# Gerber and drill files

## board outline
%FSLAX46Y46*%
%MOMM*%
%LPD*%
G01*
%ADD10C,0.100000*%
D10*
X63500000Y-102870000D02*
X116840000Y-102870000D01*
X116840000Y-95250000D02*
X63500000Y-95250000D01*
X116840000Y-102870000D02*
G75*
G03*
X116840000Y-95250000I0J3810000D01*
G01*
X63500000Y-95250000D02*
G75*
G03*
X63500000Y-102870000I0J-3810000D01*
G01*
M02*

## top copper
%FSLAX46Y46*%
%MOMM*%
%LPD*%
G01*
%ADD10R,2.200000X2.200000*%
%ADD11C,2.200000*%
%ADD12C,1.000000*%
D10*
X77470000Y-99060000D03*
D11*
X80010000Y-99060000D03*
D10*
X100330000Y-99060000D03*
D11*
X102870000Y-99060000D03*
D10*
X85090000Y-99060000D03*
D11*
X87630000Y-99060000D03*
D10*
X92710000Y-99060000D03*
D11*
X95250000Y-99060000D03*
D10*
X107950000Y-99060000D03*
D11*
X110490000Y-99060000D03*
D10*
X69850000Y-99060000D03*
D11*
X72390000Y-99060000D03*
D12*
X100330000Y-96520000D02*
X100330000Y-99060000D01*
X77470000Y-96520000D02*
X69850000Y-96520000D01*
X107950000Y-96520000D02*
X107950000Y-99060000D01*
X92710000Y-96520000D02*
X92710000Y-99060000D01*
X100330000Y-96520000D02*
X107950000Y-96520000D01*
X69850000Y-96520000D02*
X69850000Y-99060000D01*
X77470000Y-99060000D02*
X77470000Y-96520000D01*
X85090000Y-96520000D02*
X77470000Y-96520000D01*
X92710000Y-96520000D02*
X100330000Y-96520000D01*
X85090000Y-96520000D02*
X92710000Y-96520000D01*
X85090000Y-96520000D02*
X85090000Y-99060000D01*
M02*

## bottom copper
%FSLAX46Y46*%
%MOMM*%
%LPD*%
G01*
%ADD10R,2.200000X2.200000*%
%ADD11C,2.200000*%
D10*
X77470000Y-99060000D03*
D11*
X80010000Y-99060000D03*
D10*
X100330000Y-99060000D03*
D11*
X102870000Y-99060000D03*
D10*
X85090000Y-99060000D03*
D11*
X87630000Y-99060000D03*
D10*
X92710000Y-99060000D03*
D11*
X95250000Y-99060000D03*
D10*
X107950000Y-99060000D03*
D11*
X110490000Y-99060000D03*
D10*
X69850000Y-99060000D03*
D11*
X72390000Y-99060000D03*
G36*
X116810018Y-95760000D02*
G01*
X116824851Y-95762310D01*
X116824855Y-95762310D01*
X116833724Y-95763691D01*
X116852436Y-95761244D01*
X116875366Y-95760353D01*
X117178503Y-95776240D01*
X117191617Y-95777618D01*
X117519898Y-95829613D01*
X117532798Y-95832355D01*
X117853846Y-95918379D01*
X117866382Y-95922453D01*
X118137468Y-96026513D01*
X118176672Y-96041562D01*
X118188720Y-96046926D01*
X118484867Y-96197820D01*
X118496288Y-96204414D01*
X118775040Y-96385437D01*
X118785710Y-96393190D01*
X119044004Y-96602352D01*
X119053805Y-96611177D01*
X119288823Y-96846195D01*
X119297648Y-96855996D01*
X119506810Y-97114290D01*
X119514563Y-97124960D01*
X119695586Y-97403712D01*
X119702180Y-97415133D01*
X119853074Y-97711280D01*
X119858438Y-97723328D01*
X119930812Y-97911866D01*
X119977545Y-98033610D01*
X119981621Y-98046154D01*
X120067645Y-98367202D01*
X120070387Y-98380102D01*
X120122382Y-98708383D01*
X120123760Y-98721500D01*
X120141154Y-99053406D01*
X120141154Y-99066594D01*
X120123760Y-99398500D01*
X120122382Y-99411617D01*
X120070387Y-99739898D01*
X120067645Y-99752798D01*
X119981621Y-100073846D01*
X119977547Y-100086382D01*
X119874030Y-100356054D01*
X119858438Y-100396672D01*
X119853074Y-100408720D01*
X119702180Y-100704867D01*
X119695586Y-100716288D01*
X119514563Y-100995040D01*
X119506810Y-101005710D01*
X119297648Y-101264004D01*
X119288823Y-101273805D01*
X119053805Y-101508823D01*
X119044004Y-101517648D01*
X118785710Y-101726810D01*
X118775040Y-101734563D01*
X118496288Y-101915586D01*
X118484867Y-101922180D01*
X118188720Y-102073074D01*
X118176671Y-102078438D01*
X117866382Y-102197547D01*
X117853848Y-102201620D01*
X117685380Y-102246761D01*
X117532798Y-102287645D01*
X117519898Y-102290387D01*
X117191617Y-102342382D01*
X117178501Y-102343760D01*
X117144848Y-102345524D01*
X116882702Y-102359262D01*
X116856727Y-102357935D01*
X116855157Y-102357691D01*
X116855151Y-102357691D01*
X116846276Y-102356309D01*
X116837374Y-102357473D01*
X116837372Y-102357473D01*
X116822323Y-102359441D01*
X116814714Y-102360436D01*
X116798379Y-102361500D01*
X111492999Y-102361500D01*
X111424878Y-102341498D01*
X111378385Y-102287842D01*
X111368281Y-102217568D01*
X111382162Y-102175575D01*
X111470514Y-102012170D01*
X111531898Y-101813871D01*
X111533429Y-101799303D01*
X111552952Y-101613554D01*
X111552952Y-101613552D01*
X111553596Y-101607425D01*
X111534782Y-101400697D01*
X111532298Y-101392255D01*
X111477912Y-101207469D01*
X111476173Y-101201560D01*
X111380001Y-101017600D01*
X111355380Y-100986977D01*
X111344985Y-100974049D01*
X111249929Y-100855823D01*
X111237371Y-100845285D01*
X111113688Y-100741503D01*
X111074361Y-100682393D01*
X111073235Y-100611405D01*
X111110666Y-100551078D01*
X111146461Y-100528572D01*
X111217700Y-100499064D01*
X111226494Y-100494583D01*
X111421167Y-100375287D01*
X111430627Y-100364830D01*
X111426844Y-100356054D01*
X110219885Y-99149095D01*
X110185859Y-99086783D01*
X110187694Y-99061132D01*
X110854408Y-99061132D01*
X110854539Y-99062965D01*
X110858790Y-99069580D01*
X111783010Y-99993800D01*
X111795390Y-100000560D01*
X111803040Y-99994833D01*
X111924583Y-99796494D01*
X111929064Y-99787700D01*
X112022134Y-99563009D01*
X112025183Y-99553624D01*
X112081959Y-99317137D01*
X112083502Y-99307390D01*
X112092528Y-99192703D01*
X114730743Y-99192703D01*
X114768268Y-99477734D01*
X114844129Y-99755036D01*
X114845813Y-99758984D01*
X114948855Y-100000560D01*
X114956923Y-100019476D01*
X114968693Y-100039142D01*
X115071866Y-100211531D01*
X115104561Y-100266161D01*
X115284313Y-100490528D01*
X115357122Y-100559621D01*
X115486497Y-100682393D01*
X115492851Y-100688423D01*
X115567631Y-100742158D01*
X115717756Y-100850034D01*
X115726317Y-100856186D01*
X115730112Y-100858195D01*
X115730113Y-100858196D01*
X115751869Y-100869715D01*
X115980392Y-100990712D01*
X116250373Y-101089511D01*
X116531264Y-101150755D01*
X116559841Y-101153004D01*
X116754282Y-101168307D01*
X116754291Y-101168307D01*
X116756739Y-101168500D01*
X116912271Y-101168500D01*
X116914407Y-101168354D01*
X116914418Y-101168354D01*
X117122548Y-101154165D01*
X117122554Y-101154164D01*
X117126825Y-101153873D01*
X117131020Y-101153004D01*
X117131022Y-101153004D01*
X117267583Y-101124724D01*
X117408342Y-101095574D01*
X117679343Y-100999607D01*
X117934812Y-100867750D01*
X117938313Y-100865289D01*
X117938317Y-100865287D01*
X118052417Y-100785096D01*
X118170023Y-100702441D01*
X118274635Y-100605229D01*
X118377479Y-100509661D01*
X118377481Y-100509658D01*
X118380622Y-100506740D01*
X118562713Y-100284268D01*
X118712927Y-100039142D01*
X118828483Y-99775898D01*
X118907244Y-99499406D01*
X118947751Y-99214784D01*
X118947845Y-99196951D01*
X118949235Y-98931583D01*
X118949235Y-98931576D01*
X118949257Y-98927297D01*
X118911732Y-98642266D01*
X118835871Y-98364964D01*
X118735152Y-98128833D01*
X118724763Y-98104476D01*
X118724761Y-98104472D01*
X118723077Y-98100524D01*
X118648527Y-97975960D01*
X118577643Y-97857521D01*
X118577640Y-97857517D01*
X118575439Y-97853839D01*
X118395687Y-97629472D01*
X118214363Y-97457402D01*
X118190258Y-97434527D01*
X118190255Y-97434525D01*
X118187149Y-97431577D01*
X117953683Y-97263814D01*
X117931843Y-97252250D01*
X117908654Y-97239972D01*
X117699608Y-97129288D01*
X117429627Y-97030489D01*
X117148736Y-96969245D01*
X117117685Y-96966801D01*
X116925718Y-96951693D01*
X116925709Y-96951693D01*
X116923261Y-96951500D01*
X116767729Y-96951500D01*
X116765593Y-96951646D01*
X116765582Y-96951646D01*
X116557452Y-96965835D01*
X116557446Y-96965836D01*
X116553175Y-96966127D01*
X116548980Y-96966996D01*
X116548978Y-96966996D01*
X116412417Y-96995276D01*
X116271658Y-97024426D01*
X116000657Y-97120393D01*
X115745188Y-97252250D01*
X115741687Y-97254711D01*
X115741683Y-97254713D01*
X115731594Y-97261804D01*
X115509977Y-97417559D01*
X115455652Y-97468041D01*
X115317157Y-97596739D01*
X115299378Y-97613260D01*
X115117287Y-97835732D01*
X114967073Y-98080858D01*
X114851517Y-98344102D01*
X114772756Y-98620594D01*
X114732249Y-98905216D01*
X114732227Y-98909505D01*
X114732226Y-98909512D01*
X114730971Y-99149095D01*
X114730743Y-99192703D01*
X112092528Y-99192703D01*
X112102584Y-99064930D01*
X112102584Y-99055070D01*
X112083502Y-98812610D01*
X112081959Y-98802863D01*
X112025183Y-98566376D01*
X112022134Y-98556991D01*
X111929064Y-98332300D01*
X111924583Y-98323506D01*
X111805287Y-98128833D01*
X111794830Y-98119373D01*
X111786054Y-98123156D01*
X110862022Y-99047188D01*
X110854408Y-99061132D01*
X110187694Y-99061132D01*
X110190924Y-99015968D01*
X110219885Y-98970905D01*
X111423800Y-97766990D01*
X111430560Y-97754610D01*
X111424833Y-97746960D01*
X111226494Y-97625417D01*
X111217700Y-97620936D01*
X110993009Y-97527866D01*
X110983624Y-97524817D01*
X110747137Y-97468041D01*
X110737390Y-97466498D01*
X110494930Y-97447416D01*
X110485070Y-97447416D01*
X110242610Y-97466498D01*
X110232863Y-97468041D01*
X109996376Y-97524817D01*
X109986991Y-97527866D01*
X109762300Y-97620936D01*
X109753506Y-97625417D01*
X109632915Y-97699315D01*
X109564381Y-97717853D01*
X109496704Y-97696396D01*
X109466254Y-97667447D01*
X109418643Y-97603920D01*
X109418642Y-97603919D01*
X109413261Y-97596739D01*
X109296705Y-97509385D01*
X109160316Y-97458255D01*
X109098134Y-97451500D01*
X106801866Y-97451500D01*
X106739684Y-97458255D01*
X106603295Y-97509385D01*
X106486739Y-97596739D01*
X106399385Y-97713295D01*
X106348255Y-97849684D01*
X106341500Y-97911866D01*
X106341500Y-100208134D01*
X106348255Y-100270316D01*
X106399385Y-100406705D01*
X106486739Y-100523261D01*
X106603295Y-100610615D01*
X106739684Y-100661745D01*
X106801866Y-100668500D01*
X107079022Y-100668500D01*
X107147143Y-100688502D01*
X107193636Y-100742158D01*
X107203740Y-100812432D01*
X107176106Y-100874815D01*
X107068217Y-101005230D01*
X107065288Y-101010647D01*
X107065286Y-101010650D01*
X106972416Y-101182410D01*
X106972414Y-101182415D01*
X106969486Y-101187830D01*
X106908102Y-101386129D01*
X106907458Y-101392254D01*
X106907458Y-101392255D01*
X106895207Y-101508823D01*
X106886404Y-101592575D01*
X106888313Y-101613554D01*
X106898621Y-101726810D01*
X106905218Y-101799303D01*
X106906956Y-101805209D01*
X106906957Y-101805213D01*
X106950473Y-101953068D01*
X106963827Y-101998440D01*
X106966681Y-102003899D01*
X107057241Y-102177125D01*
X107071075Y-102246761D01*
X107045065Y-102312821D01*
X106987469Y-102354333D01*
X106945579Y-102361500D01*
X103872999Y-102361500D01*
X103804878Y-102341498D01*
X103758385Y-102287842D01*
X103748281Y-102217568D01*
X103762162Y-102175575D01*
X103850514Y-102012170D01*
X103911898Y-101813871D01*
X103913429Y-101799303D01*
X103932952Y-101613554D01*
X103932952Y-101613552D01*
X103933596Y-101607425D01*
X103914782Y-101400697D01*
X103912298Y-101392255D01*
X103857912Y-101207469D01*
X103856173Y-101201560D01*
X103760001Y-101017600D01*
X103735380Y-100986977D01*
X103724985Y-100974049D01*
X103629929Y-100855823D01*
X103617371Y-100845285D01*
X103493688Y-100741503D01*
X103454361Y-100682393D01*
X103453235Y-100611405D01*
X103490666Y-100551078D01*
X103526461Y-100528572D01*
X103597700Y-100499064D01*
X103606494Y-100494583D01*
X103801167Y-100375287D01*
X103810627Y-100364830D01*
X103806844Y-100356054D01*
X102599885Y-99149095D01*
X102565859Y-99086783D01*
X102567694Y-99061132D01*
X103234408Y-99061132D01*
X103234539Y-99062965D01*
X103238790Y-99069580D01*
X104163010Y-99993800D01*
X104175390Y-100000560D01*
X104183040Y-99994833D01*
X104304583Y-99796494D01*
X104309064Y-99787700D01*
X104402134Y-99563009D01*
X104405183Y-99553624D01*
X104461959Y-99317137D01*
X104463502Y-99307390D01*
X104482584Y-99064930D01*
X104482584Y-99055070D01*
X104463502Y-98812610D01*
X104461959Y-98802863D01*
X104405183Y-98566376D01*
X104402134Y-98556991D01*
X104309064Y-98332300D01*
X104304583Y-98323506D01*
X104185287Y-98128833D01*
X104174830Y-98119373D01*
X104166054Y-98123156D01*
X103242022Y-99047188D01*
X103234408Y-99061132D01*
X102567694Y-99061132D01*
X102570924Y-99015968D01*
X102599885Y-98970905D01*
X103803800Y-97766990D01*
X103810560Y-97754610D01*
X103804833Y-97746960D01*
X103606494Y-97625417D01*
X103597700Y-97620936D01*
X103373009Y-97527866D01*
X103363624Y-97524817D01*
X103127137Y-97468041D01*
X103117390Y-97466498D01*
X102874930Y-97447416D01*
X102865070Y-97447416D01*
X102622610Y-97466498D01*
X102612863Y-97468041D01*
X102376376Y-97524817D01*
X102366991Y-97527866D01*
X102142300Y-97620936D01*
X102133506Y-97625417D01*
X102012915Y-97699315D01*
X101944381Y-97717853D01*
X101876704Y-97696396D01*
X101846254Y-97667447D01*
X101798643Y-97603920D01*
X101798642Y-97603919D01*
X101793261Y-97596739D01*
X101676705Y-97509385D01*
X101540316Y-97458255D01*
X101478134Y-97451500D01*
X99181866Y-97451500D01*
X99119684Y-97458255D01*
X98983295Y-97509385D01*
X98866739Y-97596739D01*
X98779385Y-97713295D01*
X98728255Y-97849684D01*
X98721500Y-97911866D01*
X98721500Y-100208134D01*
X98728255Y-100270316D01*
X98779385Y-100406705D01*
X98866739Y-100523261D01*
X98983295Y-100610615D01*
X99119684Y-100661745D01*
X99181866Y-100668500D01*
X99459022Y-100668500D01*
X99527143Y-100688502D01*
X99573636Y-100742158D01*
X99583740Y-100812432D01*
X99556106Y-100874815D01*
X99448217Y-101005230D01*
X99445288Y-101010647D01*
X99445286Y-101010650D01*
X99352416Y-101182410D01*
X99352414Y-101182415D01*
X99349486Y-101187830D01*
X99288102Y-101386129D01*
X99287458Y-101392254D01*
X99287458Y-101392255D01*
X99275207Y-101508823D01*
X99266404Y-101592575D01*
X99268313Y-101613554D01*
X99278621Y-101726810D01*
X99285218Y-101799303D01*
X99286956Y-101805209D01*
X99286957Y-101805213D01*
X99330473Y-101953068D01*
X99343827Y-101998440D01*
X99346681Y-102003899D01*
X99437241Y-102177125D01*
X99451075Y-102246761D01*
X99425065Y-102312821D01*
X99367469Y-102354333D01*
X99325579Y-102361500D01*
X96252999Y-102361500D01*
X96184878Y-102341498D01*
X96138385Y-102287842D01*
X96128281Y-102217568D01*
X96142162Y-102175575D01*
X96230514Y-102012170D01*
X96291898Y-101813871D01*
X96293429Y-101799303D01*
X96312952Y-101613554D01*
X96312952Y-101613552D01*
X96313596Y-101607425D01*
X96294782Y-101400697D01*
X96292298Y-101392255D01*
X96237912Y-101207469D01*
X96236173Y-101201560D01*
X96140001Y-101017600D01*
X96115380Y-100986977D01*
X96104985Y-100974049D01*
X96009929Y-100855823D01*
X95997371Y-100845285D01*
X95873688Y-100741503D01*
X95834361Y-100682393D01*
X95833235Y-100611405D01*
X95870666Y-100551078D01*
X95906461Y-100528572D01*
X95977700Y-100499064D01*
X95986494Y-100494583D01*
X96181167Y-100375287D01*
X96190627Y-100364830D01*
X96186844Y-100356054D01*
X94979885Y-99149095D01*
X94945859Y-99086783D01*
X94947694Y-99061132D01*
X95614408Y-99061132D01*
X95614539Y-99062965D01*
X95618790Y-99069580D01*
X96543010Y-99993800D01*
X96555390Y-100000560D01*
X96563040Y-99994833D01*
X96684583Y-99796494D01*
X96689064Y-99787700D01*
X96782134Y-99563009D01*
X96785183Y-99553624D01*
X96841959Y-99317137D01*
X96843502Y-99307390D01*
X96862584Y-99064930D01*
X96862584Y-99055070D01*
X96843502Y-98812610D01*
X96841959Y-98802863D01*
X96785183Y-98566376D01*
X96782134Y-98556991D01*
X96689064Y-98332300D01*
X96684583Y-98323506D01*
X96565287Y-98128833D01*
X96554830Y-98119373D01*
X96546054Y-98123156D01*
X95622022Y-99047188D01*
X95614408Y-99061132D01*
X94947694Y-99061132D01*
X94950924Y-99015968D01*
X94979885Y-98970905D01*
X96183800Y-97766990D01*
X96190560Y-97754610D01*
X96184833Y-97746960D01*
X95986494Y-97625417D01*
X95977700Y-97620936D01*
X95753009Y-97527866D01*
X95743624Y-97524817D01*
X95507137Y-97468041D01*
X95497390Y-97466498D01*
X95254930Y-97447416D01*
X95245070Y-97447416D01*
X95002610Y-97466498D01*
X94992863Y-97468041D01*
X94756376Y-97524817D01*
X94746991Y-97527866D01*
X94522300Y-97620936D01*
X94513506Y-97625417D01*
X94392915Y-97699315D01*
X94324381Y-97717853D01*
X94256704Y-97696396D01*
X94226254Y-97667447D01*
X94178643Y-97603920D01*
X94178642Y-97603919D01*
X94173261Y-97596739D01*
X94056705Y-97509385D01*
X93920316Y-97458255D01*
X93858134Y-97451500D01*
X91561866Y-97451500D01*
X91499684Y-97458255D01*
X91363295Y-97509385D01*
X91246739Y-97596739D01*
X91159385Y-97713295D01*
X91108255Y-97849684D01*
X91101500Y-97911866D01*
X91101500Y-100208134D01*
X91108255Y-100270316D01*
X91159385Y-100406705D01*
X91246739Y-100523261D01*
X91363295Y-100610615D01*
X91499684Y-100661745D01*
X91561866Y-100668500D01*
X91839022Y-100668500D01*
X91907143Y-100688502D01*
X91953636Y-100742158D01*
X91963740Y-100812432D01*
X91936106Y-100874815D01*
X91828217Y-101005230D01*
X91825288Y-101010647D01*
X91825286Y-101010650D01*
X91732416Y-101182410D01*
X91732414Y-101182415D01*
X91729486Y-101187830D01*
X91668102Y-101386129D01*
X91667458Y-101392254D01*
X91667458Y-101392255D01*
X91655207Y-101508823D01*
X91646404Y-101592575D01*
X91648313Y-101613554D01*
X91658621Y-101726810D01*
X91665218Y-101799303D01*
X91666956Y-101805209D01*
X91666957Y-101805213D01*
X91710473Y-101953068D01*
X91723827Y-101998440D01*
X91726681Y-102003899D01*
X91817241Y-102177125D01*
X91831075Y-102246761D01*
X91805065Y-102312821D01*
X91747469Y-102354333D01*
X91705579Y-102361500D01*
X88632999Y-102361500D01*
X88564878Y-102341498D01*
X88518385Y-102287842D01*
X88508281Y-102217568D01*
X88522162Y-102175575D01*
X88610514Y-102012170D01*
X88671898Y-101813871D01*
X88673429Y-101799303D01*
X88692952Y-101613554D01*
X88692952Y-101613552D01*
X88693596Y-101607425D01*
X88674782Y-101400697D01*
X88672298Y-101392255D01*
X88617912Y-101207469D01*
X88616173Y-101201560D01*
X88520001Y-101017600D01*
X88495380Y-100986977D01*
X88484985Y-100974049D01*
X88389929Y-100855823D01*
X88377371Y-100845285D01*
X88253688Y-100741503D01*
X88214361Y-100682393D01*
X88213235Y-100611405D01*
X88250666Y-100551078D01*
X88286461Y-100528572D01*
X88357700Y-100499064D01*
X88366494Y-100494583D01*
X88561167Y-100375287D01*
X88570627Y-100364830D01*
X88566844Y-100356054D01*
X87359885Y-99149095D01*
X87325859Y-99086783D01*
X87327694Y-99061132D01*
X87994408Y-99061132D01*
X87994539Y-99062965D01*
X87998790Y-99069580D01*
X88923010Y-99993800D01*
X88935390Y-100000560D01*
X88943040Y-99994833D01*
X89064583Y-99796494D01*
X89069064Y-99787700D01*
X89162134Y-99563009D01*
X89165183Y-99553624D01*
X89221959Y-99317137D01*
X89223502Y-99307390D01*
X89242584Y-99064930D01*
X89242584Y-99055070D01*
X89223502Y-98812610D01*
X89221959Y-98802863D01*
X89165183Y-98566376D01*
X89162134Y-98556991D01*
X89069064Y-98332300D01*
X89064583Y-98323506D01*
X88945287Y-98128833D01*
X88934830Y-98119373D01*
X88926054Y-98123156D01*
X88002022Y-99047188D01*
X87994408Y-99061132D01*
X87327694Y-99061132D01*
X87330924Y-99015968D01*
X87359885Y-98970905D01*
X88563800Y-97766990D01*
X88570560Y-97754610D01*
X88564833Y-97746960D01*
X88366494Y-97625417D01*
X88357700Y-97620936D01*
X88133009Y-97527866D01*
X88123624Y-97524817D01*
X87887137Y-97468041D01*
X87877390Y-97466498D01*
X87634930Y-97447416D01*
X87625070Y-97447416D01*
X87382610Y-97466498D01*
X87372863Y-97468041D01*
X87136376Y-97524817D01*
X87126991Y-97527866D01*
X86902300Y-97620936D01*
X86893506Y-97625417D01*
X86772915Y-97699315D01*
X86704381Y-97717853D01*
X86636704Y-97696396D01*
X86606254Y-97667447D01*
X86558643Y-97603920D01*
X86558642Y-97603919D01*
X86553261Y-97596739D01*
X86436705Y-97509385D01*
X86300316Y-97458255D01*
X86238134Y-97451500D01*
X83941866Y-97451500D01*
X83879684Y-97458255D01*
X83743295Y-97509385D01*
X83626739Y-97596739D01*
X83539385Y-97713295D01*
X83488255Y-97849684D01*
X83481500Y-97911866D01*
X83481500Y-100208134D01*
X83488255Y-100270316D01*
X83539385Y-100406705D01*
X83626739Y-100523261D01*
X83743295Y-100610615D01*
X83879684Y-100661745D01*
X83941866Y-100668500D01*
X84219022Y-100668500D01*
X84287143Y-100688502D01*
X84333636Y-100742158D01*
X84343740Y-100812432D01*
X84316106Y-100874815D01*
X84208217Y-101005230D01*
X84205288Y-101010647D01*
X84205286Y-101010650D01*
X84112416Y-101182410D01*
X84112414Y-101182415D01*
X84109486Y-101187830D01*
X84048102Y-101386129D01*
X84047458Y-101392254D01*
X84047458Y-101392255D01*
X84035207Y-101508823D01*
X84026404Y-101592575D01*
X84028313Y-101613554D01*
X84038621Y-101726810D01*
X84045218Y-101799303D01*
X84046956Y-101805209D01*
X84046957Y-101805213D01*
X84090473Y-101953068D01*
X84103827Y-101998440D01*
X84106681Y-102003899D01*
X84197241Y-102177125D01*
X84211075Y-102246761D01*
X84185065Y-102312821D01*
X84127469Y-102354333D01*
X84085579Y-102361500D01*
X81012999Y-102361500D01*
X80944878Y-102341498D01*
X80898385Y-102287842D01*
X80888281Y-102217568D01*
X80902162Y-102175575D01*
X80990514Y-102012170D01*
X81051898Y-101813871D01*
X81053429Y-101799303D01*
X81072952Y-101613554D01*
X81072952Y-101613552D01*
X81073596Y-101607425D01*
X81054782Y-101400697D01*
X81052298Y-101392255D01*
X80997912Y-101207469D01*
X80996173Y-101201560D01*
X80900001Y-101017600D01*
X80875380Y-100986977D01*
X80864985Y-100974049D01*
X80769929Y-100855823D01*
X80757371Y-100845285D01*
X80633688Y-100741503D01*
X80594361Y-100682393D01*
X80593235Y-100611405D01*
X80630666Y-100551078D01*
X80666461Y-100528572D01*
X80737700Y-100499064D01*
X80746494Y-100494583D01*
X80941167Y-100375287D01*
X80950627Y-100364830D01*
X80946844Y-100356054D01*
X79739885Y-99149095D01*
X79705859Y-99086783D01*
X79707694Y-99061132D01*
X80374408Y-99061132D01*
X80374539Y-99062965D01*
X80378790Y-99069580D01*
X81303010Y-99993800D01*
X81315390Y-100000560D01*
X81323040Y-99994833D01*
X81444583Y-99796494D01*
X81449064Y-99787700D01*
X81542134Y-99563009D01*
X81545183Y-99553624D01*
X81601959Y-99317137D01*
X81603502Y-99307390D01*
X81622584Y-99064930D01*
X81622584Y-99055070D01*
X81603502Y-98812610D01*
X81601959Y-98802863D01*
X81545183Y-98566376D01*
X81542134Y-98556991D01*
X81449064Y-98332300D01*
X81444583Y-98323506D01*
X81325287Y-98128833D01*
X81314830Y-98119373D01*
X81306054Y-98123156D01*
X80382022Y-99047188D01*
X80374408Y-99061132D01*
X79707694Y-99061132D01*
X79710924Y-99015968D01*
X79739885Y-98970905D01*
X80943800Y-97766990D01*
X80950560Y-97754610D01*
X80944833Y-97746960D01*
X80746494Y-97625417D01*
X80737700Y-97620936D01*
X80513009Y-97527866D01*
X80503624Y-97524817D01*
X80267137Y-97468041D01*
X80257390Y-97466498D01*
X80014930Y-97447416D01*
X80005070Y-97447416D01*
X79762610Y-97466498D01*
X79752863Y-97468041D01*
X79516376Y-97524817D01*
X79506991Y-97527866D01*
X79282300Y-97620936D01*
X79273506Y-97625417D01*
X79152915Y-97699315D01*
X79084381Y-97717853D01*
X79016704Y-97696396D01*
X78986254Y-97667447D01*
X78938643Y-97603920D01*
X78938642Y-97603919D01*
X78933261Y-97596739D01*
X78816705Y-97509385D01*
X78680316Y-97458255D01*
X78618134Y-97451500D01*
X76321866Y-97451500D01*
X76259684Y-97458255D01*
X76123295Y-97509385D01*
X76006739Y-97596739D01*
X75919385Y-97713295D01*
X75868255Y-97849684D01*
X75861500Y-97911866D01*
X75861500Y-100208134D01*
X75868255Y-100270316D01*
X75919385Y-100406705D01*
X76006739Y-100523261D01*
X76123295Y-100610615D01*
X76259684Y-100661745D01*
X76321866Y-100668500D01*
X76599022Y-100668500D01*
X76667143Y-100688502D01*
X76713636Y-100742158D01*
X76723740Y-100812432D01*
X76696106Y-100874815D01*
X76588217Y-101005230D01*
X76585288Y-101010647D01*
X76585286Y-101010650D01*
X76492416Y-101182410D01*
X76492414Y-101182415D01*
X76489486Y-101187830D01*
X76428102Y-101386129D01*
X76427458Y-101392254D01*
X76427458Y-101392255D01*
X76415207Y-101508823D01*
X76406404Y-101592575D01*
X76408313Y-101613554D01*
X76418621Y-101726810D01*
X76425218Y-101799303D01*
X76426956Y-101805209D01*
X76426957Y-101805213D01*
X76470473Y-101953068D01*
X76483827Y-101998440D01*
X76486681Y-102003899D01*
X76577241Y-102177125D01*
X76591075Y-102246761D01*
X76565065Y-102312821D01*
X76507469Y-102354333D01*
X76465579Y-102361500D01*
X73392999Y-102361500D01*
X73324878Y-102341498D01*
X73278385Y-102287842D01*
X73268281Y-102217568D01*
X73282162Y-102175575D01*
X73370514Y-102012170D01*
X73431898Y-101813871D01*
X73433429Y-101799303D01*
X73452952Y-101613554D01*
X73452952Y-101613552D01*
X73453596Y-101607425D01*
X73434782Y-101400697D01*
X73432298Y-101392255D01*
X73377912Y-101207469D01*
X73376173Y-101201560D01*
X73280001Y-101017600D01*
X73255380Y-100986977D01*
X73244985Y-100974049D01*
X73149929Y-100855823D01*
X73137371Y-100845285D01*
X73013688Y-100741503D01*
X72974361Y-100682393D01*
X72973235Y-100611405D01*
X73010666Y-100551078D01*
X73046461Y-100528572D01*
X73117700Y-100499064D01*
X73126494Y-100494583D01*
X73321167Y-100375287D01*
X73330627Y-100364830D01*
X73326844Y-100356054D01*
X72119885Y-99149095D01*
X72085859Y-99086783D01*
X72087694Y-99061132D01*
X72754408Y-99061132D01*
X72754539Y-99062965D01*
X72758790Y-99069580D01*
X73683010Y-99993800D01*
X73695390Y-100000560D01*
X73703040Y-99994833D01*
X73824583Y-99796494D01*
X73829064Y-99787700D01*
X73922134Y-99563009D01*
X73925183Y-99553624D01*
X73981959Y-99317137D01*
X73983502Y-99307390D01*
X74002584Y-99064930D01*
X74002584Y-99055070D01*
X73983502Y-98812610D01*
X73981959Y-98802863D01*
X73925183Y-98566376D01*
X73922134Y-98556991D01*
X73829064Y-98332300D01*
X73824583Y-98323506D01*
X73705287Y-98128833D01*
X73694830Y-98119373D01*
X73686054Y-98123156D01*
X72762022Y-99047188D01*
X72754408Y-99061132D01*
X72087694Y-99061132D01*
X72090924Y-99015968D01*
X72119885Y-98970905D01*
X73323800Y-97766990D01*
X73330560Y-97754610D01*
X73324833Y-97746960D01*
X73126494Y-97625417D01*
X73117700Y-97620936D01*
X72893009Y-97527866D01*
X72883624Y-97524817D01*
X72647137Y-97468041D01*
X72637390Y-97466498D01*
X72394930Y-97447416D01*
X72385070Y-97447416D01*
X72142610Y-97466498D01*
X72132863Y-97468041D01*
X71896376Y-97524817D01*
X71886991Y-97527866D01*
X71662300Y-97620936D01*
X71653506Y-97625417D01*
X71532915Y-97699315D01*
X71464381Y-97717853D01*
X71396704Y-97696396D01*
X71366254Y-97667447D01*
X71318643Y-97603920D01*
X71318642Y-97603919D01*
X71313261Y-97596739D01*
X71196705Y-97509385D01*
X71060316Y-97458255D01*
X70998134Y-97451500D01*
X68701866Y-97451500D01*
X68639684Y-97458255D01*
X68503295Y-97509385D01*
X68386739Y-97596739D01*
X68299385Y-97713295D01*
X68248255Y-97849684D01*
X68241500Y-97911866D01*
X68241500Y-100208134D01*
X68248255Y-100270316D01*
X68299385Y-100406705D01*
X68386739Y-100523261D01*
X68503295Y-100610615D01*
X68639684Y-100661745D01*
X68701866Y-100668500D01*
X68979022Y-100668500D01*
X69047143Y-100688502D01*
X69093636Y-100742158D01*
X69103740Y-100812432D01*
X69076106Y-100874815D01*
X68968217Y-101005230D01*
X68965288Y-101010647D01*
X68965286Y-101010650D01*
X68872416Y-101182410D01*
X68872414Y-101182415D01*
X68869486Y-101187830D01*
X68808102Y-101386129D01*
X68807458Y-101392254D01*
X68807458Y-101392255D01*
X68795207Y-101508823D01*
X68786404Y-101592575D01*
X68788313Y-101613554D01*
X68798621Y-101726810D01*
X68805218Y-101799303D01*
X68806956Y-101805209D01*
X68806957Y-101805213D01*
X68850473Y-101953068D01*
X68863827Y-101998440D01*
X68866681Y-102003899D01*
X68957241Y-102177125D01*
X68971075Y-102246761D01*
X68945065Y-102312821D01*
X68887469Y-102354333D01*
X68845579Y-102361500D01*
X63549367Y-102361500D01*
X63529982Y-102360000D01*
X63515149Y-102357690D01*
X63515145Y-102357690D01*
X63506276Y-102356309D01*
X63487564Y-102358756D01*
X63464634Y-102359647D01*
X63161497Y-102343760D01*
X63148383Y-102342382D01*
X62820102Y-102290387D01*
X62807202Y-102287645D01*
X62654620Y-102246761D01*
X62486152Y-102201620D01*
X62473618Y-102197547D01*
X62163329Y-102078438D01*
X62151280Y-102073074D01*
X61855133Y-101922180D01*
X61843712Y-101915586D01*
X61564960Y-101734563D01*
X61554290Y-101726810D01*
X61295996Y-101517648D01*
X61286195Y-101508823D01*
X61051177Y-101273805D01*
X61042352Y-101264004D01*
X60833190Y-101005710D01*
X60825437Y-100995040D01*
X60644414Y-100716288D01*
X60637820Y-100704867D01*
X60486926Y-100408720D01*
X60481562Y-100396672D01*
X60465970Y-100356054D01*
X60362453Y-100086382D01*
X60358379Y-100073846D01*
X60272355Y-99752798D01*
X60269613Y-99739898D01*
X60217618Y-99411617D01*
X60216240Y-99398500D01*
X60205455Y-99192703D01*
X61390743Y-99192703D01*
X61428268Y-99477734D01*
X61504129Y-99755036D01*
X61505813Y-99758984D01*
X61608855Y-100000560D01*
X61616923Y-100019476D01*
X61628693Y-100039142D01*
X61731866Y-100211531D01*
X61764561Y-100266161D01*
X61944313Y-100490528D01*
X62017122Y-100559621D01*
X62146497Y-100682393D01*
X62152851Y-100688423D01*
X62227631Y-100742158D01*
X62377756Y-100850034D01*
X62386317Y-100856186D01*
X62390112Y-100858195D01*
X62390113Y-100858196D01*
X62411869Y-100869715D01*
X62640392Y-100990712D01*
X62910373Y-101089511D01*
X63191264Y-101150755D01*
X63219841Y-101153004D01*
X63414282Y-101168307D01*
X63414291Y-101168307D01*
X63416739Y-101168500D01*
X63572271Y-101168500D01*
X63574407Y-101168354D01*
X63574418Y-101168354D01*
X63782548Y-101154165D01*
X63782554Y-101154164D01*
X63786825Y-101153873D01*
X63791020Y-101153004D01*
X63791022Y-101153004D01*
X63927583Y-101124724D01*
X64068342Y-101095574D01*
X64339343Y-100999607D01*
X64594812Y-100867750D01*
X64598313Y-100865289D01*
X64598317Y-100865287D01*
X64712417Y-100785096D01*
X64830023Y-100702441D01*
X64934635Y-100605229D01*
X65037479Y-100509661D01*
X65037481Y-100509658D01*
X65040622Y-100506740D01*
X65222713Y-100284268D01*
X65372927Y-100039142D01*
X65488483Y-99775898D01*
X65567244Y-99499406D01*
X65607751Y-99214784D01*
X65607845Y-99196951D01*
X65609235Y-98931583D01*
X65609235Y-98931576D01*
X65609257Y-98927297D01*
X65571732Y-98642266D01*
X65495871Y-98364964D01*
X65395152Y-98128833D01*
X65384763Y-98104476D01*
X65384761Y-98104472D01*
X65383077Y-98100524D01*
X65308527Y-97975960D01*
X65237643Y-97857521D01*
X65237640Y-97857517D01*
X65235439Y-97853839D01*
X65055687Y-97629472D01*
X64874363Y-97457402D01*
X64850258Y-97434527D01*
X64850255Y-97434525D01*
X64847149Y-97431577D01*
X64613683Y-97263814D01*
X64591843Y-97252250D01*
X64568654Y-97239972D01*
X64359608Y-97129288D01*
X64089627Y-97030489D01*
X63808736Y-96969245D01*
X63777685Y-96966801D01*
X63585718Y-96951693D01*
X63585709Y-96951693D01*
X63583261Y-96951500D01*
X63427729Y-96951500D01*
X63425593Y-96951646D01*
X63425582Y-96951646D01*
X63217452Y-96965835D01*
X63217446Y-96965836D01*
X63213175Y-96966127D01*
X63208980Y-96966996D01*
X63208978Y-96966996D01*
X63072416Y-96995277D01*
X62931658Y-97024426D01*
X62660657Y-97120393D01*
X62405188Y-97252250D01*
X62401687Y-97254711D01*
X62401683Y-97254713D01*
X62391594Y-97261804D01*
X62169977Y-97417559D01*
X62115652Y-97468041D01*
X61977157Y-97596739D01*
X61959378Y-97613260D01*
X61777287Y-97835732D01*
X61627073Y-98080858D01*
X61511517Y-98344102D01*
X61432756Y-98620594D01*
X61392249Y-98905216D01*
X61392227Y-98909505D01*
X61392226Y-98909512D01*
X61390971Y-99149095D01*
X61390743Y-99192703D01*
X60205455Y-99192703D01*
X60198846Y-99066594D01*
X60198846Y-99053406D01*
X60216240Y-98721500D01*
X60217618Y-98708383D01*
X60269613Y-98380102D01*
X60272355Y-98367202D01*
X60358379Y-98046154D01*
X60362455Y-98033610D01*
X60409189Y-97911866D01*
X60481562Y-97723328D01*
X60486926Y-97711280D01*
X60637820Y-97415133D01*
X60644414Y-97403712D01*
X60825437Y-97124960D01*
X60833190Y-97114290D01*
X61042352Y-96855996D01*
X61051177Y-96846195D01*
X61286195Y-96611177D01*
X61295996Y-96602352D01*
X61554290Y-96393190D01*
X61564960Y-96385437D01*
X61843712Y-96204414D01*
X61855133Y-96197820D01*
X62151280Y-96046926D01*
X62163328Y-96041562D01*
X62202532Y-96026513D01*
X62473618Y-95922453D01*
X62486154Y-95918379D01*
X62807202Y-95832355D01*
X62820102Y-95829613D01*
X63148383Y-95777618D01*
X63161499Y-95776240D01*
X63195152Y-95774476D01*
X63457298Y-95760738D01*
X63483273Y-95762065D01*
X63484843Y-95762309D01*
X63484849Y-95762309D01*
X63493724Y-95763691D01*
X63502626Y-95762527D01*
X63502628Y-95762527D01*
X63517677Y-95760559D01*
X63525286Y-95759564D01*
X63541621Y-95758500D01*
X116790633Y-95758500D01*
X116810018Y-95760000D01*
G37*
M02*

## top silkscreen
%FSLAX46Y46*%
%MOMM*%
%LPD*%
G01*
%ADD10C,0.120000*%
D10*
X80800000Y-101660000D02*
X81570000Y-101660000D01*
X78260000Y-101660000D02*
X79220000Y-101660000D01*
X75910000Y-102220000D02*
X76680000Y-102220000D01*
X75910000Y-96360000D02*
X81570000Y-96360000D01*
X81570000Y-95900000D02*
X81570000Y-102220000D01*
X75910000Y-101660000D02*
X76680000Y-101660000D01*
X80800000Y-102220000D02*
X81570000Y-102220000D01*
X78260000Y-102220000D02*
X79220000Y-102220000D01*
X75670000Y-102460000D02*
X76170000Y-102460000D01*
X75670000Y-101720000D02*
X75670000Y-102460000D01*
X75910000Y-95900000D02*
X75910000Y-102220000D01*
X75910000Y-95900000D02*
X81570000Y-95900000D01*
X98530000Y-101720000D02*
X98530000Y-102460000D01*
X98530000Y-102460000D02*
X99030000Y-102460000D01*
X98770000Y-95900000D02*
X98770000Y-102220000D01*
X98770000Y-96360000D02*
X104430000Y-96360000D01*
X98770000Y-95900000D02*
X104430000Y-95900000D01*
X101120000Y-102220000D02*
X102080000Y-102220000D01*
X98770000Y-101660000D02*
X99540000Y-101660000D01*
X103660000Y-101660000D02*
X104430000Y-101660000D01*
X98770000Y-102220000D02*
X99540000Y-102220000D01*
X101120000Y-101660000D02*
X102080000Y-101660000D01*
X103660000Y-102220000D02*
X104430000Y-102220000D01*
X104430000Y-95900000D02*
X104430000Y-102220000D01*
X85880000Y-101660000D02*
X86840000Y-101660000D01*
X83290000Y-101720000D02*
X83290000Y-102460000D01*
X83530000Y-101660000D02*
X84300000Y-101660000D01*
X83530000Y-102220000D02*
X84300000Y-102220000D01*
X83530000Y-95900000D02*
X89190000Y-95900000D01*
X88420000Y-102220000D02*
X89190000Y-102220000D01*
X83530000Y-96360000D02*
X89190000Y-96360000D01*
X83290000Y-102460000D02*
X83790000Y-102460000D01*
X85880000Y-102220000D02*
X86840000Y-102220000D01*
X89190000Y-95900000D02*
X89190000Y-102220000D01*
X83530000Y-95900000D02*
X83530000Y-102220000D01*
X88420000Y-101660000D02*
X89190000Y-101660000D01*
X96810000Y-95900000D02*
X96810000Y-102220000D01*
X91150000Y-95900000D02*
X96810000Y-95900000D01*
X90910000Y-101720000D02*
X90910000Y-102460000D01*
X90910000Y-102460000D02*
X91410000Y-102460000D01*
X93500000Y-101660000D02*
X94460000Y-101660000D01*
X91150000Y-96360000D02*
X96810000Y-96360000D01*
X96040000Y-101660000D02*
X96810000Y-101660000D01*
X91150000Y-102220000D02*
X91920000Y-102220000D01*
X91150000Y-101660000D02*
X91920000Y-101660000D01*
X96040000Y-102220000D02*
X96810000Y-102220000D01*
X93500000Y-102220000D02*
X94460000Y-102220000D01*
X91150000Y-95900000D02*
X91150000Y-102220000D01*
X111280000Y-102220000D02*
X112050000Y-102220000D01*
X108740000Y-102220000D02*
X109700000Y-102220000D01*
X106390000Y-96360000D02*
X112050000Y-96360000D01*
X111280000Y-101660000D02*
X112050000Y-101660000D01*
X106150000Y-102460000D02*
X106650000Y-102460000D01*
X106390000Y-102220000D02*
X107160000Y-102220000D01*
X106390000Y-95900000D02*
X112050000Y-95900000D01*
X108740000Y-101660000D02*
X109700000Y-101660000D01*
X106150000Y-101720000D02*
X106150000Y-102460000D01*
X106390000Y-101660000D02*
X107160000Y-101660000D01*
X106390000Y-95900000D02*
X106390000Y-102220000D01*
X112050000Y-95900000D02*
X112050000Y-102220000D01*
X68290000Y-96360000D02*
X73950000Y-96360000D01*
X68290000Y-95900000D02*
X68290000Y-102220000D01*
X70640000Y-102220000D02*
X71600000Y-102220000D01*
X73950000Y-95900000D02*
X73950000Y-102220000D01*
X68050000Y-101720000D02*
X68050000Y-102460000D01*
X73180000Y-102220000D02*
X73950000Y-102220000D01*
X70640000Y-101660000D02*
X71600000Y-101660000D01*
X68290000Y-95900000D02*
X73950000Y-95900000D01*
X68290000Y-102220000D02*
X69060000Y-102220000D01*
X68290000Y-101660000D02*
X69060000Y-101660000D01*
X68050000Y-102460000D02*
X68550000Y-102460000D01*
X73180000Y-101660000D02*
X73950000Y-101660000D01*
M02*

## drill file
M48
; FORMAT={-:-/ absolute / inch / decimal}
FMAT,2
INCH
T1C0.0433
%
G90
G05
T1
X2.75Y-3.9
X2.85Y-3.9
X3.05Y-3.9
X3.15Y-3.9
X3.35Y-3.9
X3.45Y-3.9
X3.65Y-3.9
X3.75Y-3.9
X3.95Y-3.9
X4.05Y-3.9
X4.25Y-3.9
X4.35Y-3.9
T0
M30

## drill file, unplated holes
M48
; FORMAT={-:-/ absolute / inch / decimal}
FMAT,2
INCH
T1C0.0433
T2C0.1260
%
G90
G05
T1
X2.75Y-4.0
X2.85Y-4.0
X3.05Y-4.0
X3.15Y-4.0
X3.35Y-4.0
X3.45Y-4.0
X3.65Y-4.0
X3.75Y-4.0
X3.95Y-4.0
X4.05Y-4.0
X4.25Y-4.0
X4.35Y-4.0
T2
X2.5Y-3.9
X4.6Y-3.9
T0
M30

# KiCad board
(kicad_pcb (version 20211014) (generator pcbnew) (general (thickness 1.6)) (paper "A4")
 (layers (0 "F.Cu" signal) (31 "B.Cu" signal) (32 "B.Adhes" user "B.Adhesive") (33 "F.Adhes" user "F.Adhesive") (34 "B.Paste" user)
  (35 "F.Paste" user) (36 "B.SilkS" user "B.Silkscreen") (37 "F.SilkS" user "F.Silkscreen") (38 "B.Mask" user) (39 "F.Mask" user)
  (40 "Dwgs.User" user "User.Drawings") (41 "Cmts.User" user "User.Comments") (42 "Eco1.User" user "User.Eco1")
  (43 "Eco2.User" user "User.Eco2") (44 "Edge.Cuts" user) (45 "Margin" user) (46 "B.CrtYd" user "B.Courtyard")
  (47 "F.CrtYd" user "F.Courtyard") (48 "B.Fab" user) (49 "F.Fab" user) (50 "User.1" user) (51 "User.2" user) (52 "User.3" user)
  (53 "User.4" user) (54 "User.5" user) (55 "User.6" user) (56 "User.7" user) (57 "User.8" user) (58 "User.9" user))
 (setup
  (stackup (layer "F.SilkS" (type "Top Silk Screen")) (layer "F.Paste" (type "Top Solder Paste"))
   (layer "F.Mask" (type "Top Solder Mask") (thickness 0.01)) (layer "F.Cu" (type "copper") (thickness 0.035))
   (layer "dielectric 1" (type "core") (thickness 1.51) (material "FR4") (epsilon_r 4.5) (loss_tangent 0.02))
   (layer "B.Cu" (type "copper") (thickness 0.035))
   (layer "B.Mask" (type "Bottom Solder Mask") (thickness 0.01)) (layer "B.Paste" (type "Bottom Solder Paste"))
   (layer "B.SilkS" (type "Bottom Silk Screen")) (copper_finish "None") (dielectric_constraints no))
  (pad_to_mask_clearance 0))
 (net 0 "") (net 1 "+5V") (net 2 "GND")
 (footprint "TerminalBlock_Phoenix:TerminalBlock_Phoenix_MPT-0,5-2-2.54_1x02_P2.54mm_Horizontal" (layer "F.Cu") (at 77.47 99.06)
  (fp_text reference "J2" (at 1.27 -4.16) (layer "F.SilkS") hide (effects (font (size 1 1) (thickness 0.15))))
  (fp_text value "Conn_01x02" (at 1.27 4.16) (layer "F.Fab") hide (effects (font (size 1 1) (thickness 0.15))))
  (fp_line (start 3.33 2.6) (end 4.1 2.6) (layer "F.SilkS") (width 0.12))
  (fp_line (start 0.79 2.6) (end 1.75 2.6) (layer "F.SilkS") (width 0.12))
  (fp_line (start -1.56 3.16) (end -0.79 3.16) (layer "F.SilkS") (width 0.12))
  (fp_line (start -1.56 -2.7) (end 4.1 -2.7) (layer "F.SilkS") (width 0.12))
  (fp_line (start 4.1 -3.16) (end 4.1 3.16) (layer "F.SilkS") (width 0.12))
  (fp_line (start -1.56 2.6) (end -0.79 2.6) (layer "F.SilkS") (width 0.12))
  (fp_line (start 3.33 3.16) (end 4.1 3.16) (layer "F.SilkS") (width 0.12))
  (fp_line (start 0.79 3.16) (end 1.75 3.16) (layer "F.SilkS") (width 0.12))
  (fp_line (start -1.8 3.4) (end -1.3 3.4) (layer "F.SilkS") (width 0.12))
  (fp_line (start -1.8 2.66) (end -1.8 3.4) (layer "F.SilkS") (width 0.12))
  (fp_line (start -1.56 -3.16) (end -1.56 3.16) (layer "F.SilkS") (width 0.12))
  (fp_line (start -1.56 -3.16) (end 4.1 -3.16) (layer "F.SilkS") (width 0.12))
  (pad "" np_thru_hole circle (at 0 2.54) (size 1.1 1.1) (drill 1.1) (layers *.Cu *.Mask))
  (pad "" np_thru_hole circle (at 2.54 2.54) (size 1.1 1.1) (drill 1.1) (layers *.Cu *.Mask))
  (pad "1" thru_hole rect (at 0 0) (size 2.2 2.2) (drill 1.1) (layers *.Cu *.Mask) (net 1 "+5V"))
  (pad "2" thru_hole circle (at 2.54 0) (size 2.2 2.2) (drill 1.1) (layers *.Cu *.Mask) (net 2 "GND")))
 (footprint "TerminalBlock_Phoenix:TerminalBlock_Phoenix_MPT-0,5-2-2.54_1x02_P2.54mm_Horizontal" (layer "F.Cu") (at 100.33 99.06)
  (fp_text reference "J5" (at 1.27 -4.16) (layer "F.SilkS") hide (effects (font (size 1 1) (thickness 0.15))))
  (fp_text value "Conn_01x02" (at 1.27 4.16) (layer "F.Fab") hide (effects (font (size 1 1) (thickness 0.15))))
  (fp_line (start -1.8 2.66) (end -1.8 3.4) (layer "F.SilkS") (width 0.12))
  (fp_line (start -1.8 3.4) (end -1.3 3.4) (layer "F.SilkS") (width 0.12))
  (fp_line (start -1.56 -3.16) (end -1.56 3.16) (layer "F.SilkS") (width 0.12))
  (fp_line (start -1.56 -2.7) (end 4.1 -2.7) (layer "F.SilkS") (width 0.12))
  (fp_line (start -1.56 -3.16) (end 4.1 -3.16) (layer "F.SilkS") (width 0.12))
  (fp_line (start 0.79 3.16) (end 1.75 3.16) (layer "F.SilkS") (width 0.12))
  (fp_line (start -1.56 2.6) (end -0.79 2.6) (layer "F.SilkS") (width 0.12))
  (fp_line (start 3.33 2.6) (end 4.1 2.6) (layer "F.SilkS") (width 0.12))
  (fp_line (start -1.56 3.16) (end -0.79 3.16) (layer "F.SilkS") (width 0.12))
  (fp_line (start 0.79 2.6) (end 1.75 2.6) (layer "F.SilkS") (width 0.12))
  (fp_line (start 3.33 3.16) (end 4.1 3.16) (layer "F.SilkS") (width 0.12))
  (fp_line (start 4.1 -3.16) (end 4.1 3.16) (layer "F.SilkS") (width 0.12))
  (pad "" np_thru_hole circle (at 2.54 2.54) (size 1.1 1.1) (drill 1.1) (layers *.Cu *.Mask))
  (pad "" np_thru_hole circle (at 0 2.54) (size 1.1 1.1) (drill 1.1) (layers *.Cu *.Mask))
  (pad "1" thru_hole rect (at 0 0) (size 2.2 2.2) (drill 1.1) (layers *.Cu *.Mask) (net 1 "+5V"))
  (pad "2" thru_hole circle (at 2.54 0) (size 2.2 2.2) (drill 1.1) (layers *.Cu *.Mask) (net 2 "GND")))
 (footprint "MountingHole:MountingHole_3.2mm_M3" (layer "F.Cu") (at 63.5 99.06)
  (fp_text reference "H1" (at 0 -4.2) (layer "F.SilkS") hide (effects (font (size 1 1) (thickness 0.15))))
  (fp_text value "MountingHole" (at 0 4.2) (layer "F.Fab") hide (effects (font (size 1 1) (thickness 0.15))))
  (pad "" np_thru_hole circle (at 0 0) (size 3.2 3.2) (drill 3.2) (layers *.Cu *.Mask)))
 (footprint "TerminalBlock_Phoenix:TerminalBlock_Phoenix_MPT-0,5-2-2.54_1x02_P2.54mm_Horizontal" (layer "F.Cu") (at 85.09 99.06)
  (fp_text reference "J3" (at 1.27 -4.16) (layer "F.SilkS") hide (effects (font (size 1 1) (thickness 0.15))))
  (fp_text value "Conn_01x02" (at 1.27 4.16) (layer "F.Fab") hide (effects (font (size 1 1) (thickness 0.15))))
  (fp_line (start 0.79 2.6) (end 1.75 2.6) (layer "F.SilkS") (width 0.12))
  (fp_line (start -1.8 2.66) (end -1.8 3.4) (layer "F.SilkS") (width 0.12))
  (fp_line (start -1.56 2.6) (end -0.79 2.6) (layer "F.SilkS") (width 0.12))
  (fp_line (start -1.56 3.16) (end -0.79 3.16) (layer "F.SilkS") (width 0.12))
  (fp_line (start -1.56 -3.16) (end 4.1 -3.16) (layer "F.SilkS") (width 0.12))
  (fp_line (start 3.33 3.16) (end 4.1 3.16) (layer "F.SilkS") (width 0.12))
  (fp_line (start -1.56 -2.7) (end 4.1 -2.7) (layer "F.SilkS") (width 0.12))
  (fp_line (start -1.8 3.4) (end -1.3 3.4) (layer "F.SilkS") (width 0.12))
  (fp_line (start 0.79 3.16) (end 1.75 3.16) (layer "F.SilkS") (width 0.12))
  (fp_line (start 4.1 -3.16) (end 4.1 3.16) (layer "F.SilkS") (width 0.12))
  (fp_line (start -1.56 -3.16) (end -1.56 3.16) (layer "F.SilkS") (width 0.12))
  (fp_line (start 3.33 2.6) (end 4.1 2.6) (layer "F.SilkS") (width 0.12))
  (pad "" np_thru_hole circle (at 0 2.54) (size 1.1 1.1) (drill 1.1) (layers *.Cu *.Mask))
  (pad "" np_thru_hole circle (at 2.54 2.54) (size 1.1 1.1) (drill 1.1) (layers *.Cu *.Mask))
  (pad "1" thru_hole rect (at 0 0) (size 2.2 2.2) (drill 1.1) (layers *.Cu *.Mask) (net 1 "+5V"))
  (pad "2" thru_hole circle (at 2.54 0) (size 2.2 2.2) (drill 1.1) (layers *.Cu *.Mask) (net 2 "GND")))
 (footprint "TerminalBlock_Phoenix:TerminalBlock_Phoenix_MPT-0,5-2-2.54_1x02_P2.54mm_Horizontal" (layer "F.Cu") (at 92.71 99.06)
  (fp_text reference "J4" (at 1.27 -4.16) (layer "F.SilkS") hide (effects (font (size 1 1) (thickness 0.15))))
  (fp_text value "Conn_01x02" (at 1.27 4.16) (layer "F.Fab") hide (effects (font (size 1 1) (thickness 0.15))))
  (fp_line (start 4.1 -3.16) (end 4.1 3.16) (layer "F.SilkS") (width 0.12))
  (fp_line (start -1.56 -3.16) (end 4.1 -3.16) (layer "F.SilkS") (width 0.12))
  (fp_line (start -1.8 2.66) (end -1.8 3.4) (layer "F.SilkS") (width 0.12))
  (fp_line (start -1.8 3.4) (end -1.3 3.4) (layer "F.SilkS") (width 0.12))
  (fp_line (start 0.79 2.6) (end 1.75 2.6) (layer "F.SilkS") (width 0.12))
  (fp_line (start -1.56 -2.7) (end 4.1 -2.7) (layer "F.SilkS") (width 0.12))
  (fp_line (start 3.33 2.6) (end 4.1 2.6) (layer "F.SilkS") (width 0.12))
  (fp_line (start -1.56 3.16) (end -0.79 3.16) (layer "F.SilkS") (width 0.12))
  (fp_line (start -1.56 2.6) (end -0.79 2.6) (layer "F.SilkS") (width 0.12))
  (fp_line (start 3.33 3.16) (end 4.1 3.16) (layer "F.SilkS") (width 0.12))
  (fp_line (start 0.79 3.16) (end 1.75 3.16) (layer "F.SilkS") (width 0.12))
  (fp_line (start -1.56 -3.16) (end -1.56 3.16) (layer "F.SilkS") (width 0.12))
  (pad "" np_thru_hole circle (at 2.54 2.54) (size 1.1 1.1) (drill 1.1) (layers *.Cu *.Mask))
  (pad "" np_thru_hole circle (at 0 2.54) (size 1.1 1.1) (drill 1.1) (layers *.Cu *.Mask))
  (pad "1" thru_hole rect (at 0 0) (size 2.2 2.2) (drill 1.1) (layers *.Cu *.Mask) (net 1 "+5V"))
  (pad "2" thru_hole circle (at 2.54 0) (size 2.2 2.2) (drill 1.1) (layers *.Cu *.Mask) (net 2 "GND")))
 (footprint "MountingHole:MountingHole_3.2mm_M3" (layer "F.Cu") (at 116.84 99.06)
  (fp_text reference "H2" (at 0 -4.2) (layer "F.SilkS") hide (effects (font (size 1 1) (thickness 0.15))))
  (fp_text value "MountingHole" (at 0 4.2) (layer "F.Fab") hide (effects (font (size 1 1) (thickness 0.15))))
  (pad "" np_thru_hole circle (at 0 0) (size 3.2 3.2) (drill 3.2) (layers *.Cu *.Mask)))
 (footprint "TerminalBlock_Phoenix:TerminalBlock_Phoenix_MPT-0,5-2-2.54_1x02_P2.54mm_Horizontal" (layer "F.Cu") (at 107.95 99.06)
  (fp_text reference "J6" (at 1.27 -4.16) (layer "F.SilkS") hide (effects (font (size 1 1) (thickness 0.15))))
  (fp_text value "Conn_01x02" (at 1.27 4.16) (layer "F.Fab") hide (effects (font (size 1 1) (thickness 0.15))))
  (fp_line (start 3.33 3.16) (end 4.1 3.16) (layer "F.SilkS") (width 0.12))
  (fp_line (start 0.79 3.16) (end 1.75 3.16) (layer "F.SilkS") (width 0.12))
  (fp_line (start -1.56 -2.7) (end 4.1 -2.7) (layer "F.SilkS") (width 0.12))
  (fp_line (start 3.33 2.6) (end 4.1 2.6) (layer "F.SilkS") (width 0.12))
  (fp_line (start -1.8 3.4) (end -1.3 3.4) (layer "F.SilkS") (width 0.12))
  (fp_line (start -1.56 3.16) (end -0.79 3.16) (layer "F.SilkS") (width 0.12))
  (fp_line (start -1.56 -3.16) (end 4.1 -3.16) (layer "F.SilkS") (width 0.12))
  (fp_line (start 0.79 2.6) (end 1.75 2.6) (layer "F.SilkS") (width 0.12))
  (fp_line (start -1.8 2.66) (end -1.8 3.4) (layer "F.SilkS") (width 0.12))
  (fp_line (start -1.56 2.6) (end -0.79 2.6) (layer "F.SilkS") (width 0.12))
  (fp_line (start -1.56 -3.16) (end -1.56 3.16) (layer "F.SilkS") (width 0.12))
  (fp_line (start 4.1 -3.16) (end 4.1 3.16) (layer "F.SilkS") (width 0.12))
  (pad "" np_thru_hole circle (at 0 2.54) (size 1.1 1.1) (drill 1.1) (layers *.Cu *.Mask))
  (pad "" np_thru_hole circle (at 2.54 2.54) (size 1.1 1.1) (drill 1.1) (layers *.Cu *.Mask))
  (pad "1" thru_hole rect (at 0 0) (size 2.2 2.2) (drill 1.1) (layers *.Cu *.Mask) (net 1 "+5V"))
  (pad "2" thru_hole circle (at 2.54 0) (size 2.2 2.2) (drill 1.1) (layers *.Cu *.Mask) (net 2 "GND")))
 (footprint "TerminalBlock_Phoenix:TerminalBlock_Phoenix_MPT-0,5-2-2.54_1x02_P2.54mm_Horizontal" (layer "F.Cu") (at 69.85 99.06)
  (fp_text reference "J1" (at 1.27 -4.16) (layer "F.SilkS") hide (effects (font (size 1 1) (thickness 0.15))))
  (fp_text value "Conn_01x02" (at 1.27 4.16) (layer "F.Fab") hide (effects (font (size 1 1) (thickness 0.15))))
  (fp_line (start -1.56 -2.7) (end 4.1 -2.7) (layer "F.SilkS") (width 0.12))
  (fp_line (start -1.56 -3.16) (end -1.56 3.16) (layer "F.SilkS") (width 0.12))
  (fp_line (start 0.79 3.16) (end 1.75 3.16) (layer "F.SilkS") (width 0.12))
  (fp_line (start 4.1 -3.16) (end 4.1 3.16) (layer "F.SilkS") (width 0.12))
  (fp_line (start -1.8 2.66) (end -1.8 3.4) (layer "F.SilkS") (width 0.12))
  (fp_line (start 3.33 3.16) (end 4.1 3.16) (layer "F.SilkS") (width 0.12))
  (fp_line (start 0.79 2.6) (end 1.75 2.6) (layer "F.SilkS") (width 0.12))
  (fp_line (start -1.56 -3.16) (end 4.1 -3.16) (layer "F.SilkS") (width 0.12))
  (fp_line (start -1.56 3.16) (end -0.79 3.16) (layer "F.SilkS") (width 0.12))
  (fp_line (start -1.56 2.6) (end -0.79 2.6) (layer "F.SilkS") (width 0.12))
  (fp_line (start -1.8 3.4) (end -1.3 3.4) (layer "F.SilkS") (width 0.12))
  (fp_line (start 3.33 2.6) (end 4.1 2.6) (layer "F.SilkS") (width 0.12))
  (pad "" np_thru_hole circle (at 0 2.54) (size 1.1 1.1) (drill 1.1) (layers *.Cu *.Mask))
  (pad "" np_thru_hole circle (at 2.54 2.54) (size 1.1 1.1) (drill 1.1) (layers *.Cu *.Mask))
  (pad "1" thru_hole rect (at 0 0) (size 2.2 2.2) (drill 1.1) (layers *.Cu *.Mask) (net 1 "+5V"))
  (pad "2" thru_hole circle (at 2.54 0) (size 2.2 2.2) (drill 1.1) (layers *.Cu *.Mask) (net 2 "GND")))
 (gr_line (start 63.5 102.87) (end 116.84 102.87) (layer "Edge.Cuts") (width 0.1))
 (gr_line (start 116.84 95.25) (end 63.5 95.25) (layer "Edge.Cuts") (width 0.1))
 (gr_arc (start 116.84 95.25) (mid 120.65 99.06) (end 116.84 102.87) (layer "Edge.Cuts") (width 0.1))
 (gr_arc (start 63.5 102.87) (mid 59.69 99.06) (end 63.5 95.25) (layer "Edge.Cuts") (width 0.1))
 (segment (start 100.33 96.52) (end 100.33 99.06) (width 1) (layer "F.Cu") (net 1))
 (segment (start 77.47 96.52) (end 69.85 96.52) (width 1) (layer "F.Cu") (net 1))
 (segment (start 107.95 96.52) (end 107.95 99.06) (width 1) (layer "F.Cu") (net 1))
 (segment (start 92.71 96.52) (end 92.71 99.06) (width 1) (layer "F.Cu") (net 1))
 (segment (start 100.33 96.52) (end 107.95 96.52) (width 1) (layer "F.Cu") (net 1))
 (segment (start 69.85 96.52) (end 69.85 99.06) (width 1) (layer "F.Cu") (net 1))
 (segment (start 77.47 99.06) (end 77.47 96.52) (width 1) (layer "F.Cu") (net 1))
 (segment (start 85.09 96.52) (end 77.47 96.52) (width 1) (layer "F.Cu") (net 1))
 (segment (start 92.71 96.52) (end 100.33 96.52) (width 1) (layer "F.Cu") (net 1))
 (segment (start 85.09 96.52) (end 92.71 96.52) (width 1) (layer "F.Cu") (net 1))
 (segment (start 85.09 96.52) (end 85.09 99.06) (width 1) (layer "F.Cu") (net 1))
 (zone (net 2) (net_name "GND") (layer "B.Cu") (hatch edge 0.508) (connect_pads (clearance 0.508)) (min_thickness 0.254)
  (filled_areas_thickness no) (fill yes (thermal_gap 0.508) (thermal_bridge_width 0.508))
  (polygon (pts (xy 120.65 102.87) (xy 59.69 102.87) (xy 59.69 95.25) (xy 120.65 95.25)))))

